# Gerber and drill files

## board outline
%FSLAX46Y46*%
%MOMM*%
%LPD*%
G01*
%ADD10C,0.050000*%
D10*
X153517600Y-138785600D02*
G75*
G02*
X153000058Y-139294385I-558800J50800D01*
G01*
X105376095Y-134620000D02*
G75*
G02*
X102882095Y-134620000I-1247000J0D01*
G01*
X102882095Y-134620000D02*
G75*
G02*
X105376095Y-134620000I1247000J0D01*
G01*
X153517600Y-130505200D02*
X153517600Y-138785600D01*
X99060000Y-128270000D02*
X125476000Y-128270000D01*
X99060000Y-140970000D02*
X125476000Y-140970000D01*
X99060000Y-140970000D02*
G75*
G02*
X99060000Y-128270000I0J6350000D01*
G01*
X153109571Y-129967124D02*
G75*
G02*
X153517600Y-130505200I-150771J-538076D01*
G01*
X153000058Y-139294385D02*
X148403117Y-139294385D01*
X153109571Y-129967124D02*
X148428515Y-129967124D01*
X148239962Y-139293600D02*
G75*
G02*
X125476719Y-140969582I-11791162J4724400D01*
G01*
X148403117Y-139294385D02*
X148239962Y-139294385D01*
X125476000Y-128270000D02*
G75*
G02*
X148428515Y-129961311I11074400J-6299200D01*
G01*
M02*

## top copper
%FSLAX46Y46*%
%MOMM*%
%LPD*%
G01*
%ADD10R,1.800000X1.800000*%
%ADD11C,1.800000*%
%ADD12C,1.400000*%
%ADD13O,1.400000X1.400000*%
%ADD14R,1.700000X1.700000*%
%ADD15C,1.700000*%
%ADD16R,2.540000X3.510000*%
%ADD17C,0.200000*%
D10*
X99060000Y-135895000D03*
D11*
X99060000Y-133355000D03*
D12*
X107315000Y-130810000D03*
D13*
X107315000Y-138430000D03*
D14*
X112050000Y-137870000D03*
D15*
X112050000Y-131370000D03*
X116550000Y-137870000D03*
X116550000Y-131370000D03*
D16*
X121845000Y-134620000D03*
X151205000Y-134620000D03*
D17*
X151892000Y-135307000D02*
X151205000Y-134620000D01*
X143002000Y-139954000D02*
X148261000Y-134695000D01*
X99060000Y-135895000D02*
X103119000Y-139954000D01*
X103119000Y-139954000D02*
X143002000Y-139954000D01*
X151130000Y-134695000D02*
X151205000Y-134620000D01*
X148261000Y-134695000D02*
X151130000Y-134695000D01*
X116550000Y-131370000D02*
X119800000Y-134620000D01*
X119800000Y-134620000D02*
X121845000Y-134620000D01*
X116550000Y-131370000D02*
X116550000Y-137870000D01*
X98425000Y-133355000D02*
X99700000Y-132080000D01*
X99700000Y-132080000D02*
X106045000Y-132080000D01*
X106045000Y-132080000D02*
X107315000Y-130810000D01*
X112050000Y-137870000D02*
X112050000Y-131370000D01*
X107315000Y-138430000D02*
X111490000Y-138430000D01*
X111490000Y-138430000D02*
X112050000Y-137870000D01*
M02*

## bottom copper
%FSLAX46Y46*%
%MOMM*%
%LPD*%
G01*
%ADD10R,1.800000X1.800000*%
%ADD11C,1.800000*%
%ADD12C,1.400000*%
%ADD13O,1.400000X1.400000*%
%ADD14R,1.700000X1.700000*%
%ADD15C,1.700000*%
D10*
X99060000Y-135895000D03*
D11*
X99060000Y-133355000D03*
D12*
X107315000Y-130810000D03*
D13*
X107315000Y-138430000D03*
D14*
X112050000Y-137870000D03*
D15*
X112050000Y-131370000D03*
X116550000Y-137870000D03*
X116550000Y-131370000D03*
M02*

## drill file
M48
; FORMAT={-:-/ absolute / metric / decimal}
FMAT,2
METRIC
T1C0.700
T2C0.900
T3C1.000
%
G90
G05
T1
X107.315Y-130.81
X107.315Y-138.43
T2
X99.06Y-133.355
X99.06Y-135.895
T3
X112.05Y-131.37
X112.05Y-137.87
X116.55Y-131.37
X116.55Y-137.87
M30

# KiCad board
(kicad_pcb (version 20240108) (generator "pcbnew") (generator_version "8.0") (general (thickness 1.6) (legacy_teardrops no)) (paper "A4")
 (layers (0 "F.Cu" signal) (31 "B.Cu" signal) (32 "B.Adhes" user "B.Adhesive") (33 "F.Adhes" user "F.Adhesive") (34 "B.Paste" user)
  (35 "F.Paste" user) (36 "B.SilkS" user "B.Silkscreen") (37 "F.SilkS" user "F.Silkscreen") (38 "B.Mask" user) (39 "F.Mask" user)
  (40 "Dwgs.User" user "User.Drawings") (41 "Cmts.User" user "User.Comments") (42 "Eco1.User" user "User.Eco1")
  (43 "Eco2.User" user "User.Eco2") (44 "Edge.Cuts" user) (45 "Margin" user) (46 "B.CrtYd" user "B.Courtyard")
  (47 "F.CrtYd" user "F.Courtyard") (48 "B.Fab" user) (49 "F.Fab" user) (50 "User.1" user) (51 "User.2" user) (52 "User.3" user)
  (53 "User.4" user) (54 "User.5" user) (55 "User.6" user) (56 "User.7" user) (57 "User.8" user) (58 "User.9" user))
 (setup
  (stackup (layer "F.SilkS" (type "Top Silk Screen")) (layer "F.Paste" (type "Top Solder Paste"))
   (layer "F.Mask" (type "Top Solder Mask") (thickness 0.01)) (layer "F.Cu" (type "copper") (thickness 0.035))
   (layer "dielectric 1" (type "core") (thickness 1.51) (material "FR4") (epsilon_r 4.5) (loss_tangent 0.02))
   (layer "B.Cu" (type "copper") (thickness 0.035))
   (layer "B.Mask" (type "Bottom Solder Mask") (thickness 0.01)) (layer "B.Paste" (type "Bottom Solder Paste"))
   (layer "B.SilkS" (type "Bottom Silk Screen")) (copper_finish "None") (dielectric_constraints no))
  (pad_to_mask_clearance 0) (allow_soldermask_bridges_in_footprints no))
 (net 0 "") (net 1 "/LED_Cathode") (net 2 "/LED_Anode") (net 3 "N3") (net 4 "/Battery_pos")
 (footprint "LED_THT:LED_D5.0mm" (layer "F.Cu") (at 99.06 135.895 90)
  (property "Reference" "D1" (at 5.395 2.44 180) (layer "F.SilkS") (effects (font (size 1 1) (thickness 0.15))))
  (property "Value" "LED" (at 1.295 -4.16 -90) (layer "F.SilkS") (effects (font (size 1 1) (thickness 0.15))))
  (pad "1" thru_hole rect (at 0 0 90) (size 1.8 1.8) (drill 0.9) (layers "*.Cu" "*.Mask") (remove_unused_layers no) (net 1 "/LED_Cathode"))
  (pad "2" thru_hole circle (at 2.54 0 90) (size 1.8 1.8) (drill 0.9) (layers "*.Cu" "*.Mask") (remove_unused_layers no)
   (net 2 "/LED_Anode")))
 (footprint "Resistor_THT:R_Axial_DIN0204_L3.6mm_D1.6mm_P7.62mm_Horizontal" (layer "F.Cu") (at 107.315 130.81 -90)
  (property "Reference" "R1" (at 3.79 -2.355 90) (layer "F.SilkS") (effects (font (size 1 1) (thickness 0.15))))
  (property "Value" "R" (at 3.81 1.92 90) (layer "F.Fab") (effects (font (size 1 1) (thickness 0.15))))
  (pad "1" thru_hole circle (at 0 0 270) (size 1.4 1.4) (drill 0.7) (layers "*.Cu" "*.Mask") (remove_unused_layers no) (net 2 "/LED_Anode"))
  (pad "2" thru_hole oval (at 7.62 0 270) (size 1.4 1.4) (drill 0.7) (layers "*.Cu" "*.Mask") (remove_unused_layers no) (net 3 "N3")))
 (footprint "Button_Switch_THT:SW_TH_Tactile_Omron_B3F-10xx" (layer "F.Cu") (at 112.05 137.87 90)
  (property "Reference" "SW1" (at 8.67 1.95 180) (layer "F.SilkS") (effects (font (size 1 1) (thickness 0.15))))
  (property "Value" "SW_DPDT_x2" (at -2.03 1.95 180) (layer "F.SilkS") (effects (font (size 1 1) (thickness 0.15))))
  (pad "1" thru_hole rect (at 0 0 90) (size 1.7 1.7) (drill 1) (layers "*.Cu" "*.Mask") (remove_unused_layers no) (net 3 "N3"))
  (pad "1" thru_hole circle (at 6.5 0 90) (size 1.7 1.7) (drill 1) (layers "*.Cu" "*.Mask") (remove_unused_layers no) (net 3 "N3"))
  (pad "2" thru_hole circle (at 0 4.5 90) (size 1.7 1.7) (drill 1) (layers "*.Cu" "*.Mask") (remove_unused_layers no) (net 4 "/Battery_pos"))
  (pad "2" thru_hole circle (at 6.5 4.5 90) (size 1.7 1.7) (drill 1) (layers "*.Cu" "*.Mask") (remove_unused_layers no)
   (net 4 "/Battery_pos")))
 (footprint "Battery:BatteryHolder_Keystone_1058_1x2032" (layer "F.Cu") (at 136.525 134.62)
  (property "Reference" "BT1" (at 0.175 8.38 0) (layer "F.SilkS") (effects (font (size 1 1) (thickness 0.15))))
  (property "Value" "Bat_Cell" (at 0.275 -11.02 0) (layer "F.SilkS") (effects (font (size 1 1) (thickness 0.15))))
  (pad "1" smd rect (at -14.68 0) (size 2.54 3.51) (layers "F.Cu" "F.Paste" "F.Mask") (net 4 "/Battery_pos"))
  (pad "2" smd rect (at 14.68 0) (size 2.54 3.51) (layers "F.Cu" "F.Paste" "F.Mask") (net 1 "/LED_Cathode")))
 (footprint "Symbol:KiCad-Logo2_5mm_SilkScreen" (layer "B.Cu") (at 136.525 130.175 180)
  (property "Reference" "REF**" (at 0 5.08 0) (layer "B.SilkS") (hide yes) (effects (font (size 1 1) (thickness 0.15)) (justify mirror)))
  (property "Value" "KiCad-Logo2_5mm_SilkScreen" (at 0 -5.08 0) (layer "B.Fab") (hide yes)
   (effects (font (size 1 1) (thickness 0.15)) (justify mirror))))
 (gr_arc (start 153.5176 138.7856) (mid 153.352161 139.134931) (end 153.000058 139.294385) (locked yes) (stroke (width 0.05) (type default))
  (layer "Edge.Cuts"))
 (gr_circle (center 104.129095 134.62) (end 104.129095 133.373) (stroke (width 0.05) (type default)) (fill none) (layer "Edge.Cuts"))
 (gr_line (start 153.5176 130.5052) (end 153.5176 138.7856) (locked yes) (stroke (width 0.05) (type default)) (layer "Edge.Cuts"))
 (gr_line (start 99.06 128.27) (end 125.476 128.27) (locked yes) (stroke (width 0.05) (type default)) (layer "Edge.Cuts"))
 (gr_line (start 99.06 140.97) (end 125.476 140.97) (locked yes) (stroke (width 0.05) (type default)) (layer "Edge.Cuts"))
 (gr_arc (start 99.06 140.97) (mid 92.71 134.62) (end 99.06 128.27) (locked yes) (stroke (width 0.05) (type default)) (layer "Edge.Cuts"))
 (gr_arc (start 153.109571 129.967124) (mid 153.404058 130.167556) (end 153.5176 130.5052) (locked yes) (stroke (width 0.05) (type default))
  (layer "Edge.Cuts"))
 (gr_line (start 153.000058 139.294385) (end 148.403117 139.294385) (locked yes) (stroke (width 0.05) (type default)) (layer "Edge.Cuts"))
 (gr_line (start 153.109571 129.967124) (end 148.428515 129.967124) (locked yes) (stroke (width 0.05) (type default)) (layer "Edge.Cuts"))
 (gr_arc (start 148.239962 139.2936) (mid 137.381512 147.237329) (end 125.476719 140.969582) (locked yes)
  (stroke (width 0.05) (type default)) (layer "Edge.Cuts"))
 (gr_line (start 148.403117 139.294385) (end 148.239962 139.294385) (locked yes) (stroke (width 0.05) (type default)) (layer "Edge.Cuts"))
 (gr_arc (start 125.476 128.27) (mid 137.486681 121.863074) (end 148.428515 129.961311) (locked yes) (stroke (width 0.05) (type default))
  (layer "Edge.Cuts"))
 (segment (start 151.892 135.307) (end 151.205 134.62) (width 0.2) (layer "F.Cu") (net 1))
 (segment (start 143.002 139.954) (end 148.261 134.695) (width 0.2) (layer "F.Cu") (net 1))
 (segment (start 99.06 135.895) (end 103.119 139.954) (width 0.2) (layer "F.Cu") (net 1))
 (segment (start 103.119 139.954) (end 143.002 139.954) (width 0.2) (layer "F.Cu") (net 1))
 (segment (start 151.13 134.695) (end 151.205 134.62) (width 0.2) (layer "F.Cu") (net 1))
 (segment (start 148.261 134.695) (end 151.13 134.695) (width 0.2) (layer "F.Cu") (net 1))
 (segment (start 116.55 131.37) (end 119.8 134.62) (width 0.2) (layer "F.Cu") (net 4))
 (segment (start 119.8 134.62) (end 121.845 134.62) (width 0.2) (layer "F.Cu") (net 4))
 (segment (start 116.55 131.37) (end 116.55 137.87) (width 0.2) (layer "F.Cu") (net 4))
 (segment (start 98.425 133.355) (end 99.7 132.08) (width 0.2) (layer "F.Cu") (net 2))
 (segment (start 99.7 132.08) (end 106.045 132.08) (width 0.2) (layer "F.Cu") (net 2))
 (segment (start 106.045 132.08) (end 107.315 130.81) (width 0.2) (layer "F.Cu") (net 2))
 (segment (start 112.05 137.87) (end 112.05 131.37) (width 0.2) (layer "F.Cu") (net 3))
 (segment (start 107.315 138.43) (end 111.49 138.43) (width 0.2) (layer "F.Cu") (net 3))
 (segment (start 111.49 138.43) (end 112.05 137.87) (width 0.2) (layer "F.Cu") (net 3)))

